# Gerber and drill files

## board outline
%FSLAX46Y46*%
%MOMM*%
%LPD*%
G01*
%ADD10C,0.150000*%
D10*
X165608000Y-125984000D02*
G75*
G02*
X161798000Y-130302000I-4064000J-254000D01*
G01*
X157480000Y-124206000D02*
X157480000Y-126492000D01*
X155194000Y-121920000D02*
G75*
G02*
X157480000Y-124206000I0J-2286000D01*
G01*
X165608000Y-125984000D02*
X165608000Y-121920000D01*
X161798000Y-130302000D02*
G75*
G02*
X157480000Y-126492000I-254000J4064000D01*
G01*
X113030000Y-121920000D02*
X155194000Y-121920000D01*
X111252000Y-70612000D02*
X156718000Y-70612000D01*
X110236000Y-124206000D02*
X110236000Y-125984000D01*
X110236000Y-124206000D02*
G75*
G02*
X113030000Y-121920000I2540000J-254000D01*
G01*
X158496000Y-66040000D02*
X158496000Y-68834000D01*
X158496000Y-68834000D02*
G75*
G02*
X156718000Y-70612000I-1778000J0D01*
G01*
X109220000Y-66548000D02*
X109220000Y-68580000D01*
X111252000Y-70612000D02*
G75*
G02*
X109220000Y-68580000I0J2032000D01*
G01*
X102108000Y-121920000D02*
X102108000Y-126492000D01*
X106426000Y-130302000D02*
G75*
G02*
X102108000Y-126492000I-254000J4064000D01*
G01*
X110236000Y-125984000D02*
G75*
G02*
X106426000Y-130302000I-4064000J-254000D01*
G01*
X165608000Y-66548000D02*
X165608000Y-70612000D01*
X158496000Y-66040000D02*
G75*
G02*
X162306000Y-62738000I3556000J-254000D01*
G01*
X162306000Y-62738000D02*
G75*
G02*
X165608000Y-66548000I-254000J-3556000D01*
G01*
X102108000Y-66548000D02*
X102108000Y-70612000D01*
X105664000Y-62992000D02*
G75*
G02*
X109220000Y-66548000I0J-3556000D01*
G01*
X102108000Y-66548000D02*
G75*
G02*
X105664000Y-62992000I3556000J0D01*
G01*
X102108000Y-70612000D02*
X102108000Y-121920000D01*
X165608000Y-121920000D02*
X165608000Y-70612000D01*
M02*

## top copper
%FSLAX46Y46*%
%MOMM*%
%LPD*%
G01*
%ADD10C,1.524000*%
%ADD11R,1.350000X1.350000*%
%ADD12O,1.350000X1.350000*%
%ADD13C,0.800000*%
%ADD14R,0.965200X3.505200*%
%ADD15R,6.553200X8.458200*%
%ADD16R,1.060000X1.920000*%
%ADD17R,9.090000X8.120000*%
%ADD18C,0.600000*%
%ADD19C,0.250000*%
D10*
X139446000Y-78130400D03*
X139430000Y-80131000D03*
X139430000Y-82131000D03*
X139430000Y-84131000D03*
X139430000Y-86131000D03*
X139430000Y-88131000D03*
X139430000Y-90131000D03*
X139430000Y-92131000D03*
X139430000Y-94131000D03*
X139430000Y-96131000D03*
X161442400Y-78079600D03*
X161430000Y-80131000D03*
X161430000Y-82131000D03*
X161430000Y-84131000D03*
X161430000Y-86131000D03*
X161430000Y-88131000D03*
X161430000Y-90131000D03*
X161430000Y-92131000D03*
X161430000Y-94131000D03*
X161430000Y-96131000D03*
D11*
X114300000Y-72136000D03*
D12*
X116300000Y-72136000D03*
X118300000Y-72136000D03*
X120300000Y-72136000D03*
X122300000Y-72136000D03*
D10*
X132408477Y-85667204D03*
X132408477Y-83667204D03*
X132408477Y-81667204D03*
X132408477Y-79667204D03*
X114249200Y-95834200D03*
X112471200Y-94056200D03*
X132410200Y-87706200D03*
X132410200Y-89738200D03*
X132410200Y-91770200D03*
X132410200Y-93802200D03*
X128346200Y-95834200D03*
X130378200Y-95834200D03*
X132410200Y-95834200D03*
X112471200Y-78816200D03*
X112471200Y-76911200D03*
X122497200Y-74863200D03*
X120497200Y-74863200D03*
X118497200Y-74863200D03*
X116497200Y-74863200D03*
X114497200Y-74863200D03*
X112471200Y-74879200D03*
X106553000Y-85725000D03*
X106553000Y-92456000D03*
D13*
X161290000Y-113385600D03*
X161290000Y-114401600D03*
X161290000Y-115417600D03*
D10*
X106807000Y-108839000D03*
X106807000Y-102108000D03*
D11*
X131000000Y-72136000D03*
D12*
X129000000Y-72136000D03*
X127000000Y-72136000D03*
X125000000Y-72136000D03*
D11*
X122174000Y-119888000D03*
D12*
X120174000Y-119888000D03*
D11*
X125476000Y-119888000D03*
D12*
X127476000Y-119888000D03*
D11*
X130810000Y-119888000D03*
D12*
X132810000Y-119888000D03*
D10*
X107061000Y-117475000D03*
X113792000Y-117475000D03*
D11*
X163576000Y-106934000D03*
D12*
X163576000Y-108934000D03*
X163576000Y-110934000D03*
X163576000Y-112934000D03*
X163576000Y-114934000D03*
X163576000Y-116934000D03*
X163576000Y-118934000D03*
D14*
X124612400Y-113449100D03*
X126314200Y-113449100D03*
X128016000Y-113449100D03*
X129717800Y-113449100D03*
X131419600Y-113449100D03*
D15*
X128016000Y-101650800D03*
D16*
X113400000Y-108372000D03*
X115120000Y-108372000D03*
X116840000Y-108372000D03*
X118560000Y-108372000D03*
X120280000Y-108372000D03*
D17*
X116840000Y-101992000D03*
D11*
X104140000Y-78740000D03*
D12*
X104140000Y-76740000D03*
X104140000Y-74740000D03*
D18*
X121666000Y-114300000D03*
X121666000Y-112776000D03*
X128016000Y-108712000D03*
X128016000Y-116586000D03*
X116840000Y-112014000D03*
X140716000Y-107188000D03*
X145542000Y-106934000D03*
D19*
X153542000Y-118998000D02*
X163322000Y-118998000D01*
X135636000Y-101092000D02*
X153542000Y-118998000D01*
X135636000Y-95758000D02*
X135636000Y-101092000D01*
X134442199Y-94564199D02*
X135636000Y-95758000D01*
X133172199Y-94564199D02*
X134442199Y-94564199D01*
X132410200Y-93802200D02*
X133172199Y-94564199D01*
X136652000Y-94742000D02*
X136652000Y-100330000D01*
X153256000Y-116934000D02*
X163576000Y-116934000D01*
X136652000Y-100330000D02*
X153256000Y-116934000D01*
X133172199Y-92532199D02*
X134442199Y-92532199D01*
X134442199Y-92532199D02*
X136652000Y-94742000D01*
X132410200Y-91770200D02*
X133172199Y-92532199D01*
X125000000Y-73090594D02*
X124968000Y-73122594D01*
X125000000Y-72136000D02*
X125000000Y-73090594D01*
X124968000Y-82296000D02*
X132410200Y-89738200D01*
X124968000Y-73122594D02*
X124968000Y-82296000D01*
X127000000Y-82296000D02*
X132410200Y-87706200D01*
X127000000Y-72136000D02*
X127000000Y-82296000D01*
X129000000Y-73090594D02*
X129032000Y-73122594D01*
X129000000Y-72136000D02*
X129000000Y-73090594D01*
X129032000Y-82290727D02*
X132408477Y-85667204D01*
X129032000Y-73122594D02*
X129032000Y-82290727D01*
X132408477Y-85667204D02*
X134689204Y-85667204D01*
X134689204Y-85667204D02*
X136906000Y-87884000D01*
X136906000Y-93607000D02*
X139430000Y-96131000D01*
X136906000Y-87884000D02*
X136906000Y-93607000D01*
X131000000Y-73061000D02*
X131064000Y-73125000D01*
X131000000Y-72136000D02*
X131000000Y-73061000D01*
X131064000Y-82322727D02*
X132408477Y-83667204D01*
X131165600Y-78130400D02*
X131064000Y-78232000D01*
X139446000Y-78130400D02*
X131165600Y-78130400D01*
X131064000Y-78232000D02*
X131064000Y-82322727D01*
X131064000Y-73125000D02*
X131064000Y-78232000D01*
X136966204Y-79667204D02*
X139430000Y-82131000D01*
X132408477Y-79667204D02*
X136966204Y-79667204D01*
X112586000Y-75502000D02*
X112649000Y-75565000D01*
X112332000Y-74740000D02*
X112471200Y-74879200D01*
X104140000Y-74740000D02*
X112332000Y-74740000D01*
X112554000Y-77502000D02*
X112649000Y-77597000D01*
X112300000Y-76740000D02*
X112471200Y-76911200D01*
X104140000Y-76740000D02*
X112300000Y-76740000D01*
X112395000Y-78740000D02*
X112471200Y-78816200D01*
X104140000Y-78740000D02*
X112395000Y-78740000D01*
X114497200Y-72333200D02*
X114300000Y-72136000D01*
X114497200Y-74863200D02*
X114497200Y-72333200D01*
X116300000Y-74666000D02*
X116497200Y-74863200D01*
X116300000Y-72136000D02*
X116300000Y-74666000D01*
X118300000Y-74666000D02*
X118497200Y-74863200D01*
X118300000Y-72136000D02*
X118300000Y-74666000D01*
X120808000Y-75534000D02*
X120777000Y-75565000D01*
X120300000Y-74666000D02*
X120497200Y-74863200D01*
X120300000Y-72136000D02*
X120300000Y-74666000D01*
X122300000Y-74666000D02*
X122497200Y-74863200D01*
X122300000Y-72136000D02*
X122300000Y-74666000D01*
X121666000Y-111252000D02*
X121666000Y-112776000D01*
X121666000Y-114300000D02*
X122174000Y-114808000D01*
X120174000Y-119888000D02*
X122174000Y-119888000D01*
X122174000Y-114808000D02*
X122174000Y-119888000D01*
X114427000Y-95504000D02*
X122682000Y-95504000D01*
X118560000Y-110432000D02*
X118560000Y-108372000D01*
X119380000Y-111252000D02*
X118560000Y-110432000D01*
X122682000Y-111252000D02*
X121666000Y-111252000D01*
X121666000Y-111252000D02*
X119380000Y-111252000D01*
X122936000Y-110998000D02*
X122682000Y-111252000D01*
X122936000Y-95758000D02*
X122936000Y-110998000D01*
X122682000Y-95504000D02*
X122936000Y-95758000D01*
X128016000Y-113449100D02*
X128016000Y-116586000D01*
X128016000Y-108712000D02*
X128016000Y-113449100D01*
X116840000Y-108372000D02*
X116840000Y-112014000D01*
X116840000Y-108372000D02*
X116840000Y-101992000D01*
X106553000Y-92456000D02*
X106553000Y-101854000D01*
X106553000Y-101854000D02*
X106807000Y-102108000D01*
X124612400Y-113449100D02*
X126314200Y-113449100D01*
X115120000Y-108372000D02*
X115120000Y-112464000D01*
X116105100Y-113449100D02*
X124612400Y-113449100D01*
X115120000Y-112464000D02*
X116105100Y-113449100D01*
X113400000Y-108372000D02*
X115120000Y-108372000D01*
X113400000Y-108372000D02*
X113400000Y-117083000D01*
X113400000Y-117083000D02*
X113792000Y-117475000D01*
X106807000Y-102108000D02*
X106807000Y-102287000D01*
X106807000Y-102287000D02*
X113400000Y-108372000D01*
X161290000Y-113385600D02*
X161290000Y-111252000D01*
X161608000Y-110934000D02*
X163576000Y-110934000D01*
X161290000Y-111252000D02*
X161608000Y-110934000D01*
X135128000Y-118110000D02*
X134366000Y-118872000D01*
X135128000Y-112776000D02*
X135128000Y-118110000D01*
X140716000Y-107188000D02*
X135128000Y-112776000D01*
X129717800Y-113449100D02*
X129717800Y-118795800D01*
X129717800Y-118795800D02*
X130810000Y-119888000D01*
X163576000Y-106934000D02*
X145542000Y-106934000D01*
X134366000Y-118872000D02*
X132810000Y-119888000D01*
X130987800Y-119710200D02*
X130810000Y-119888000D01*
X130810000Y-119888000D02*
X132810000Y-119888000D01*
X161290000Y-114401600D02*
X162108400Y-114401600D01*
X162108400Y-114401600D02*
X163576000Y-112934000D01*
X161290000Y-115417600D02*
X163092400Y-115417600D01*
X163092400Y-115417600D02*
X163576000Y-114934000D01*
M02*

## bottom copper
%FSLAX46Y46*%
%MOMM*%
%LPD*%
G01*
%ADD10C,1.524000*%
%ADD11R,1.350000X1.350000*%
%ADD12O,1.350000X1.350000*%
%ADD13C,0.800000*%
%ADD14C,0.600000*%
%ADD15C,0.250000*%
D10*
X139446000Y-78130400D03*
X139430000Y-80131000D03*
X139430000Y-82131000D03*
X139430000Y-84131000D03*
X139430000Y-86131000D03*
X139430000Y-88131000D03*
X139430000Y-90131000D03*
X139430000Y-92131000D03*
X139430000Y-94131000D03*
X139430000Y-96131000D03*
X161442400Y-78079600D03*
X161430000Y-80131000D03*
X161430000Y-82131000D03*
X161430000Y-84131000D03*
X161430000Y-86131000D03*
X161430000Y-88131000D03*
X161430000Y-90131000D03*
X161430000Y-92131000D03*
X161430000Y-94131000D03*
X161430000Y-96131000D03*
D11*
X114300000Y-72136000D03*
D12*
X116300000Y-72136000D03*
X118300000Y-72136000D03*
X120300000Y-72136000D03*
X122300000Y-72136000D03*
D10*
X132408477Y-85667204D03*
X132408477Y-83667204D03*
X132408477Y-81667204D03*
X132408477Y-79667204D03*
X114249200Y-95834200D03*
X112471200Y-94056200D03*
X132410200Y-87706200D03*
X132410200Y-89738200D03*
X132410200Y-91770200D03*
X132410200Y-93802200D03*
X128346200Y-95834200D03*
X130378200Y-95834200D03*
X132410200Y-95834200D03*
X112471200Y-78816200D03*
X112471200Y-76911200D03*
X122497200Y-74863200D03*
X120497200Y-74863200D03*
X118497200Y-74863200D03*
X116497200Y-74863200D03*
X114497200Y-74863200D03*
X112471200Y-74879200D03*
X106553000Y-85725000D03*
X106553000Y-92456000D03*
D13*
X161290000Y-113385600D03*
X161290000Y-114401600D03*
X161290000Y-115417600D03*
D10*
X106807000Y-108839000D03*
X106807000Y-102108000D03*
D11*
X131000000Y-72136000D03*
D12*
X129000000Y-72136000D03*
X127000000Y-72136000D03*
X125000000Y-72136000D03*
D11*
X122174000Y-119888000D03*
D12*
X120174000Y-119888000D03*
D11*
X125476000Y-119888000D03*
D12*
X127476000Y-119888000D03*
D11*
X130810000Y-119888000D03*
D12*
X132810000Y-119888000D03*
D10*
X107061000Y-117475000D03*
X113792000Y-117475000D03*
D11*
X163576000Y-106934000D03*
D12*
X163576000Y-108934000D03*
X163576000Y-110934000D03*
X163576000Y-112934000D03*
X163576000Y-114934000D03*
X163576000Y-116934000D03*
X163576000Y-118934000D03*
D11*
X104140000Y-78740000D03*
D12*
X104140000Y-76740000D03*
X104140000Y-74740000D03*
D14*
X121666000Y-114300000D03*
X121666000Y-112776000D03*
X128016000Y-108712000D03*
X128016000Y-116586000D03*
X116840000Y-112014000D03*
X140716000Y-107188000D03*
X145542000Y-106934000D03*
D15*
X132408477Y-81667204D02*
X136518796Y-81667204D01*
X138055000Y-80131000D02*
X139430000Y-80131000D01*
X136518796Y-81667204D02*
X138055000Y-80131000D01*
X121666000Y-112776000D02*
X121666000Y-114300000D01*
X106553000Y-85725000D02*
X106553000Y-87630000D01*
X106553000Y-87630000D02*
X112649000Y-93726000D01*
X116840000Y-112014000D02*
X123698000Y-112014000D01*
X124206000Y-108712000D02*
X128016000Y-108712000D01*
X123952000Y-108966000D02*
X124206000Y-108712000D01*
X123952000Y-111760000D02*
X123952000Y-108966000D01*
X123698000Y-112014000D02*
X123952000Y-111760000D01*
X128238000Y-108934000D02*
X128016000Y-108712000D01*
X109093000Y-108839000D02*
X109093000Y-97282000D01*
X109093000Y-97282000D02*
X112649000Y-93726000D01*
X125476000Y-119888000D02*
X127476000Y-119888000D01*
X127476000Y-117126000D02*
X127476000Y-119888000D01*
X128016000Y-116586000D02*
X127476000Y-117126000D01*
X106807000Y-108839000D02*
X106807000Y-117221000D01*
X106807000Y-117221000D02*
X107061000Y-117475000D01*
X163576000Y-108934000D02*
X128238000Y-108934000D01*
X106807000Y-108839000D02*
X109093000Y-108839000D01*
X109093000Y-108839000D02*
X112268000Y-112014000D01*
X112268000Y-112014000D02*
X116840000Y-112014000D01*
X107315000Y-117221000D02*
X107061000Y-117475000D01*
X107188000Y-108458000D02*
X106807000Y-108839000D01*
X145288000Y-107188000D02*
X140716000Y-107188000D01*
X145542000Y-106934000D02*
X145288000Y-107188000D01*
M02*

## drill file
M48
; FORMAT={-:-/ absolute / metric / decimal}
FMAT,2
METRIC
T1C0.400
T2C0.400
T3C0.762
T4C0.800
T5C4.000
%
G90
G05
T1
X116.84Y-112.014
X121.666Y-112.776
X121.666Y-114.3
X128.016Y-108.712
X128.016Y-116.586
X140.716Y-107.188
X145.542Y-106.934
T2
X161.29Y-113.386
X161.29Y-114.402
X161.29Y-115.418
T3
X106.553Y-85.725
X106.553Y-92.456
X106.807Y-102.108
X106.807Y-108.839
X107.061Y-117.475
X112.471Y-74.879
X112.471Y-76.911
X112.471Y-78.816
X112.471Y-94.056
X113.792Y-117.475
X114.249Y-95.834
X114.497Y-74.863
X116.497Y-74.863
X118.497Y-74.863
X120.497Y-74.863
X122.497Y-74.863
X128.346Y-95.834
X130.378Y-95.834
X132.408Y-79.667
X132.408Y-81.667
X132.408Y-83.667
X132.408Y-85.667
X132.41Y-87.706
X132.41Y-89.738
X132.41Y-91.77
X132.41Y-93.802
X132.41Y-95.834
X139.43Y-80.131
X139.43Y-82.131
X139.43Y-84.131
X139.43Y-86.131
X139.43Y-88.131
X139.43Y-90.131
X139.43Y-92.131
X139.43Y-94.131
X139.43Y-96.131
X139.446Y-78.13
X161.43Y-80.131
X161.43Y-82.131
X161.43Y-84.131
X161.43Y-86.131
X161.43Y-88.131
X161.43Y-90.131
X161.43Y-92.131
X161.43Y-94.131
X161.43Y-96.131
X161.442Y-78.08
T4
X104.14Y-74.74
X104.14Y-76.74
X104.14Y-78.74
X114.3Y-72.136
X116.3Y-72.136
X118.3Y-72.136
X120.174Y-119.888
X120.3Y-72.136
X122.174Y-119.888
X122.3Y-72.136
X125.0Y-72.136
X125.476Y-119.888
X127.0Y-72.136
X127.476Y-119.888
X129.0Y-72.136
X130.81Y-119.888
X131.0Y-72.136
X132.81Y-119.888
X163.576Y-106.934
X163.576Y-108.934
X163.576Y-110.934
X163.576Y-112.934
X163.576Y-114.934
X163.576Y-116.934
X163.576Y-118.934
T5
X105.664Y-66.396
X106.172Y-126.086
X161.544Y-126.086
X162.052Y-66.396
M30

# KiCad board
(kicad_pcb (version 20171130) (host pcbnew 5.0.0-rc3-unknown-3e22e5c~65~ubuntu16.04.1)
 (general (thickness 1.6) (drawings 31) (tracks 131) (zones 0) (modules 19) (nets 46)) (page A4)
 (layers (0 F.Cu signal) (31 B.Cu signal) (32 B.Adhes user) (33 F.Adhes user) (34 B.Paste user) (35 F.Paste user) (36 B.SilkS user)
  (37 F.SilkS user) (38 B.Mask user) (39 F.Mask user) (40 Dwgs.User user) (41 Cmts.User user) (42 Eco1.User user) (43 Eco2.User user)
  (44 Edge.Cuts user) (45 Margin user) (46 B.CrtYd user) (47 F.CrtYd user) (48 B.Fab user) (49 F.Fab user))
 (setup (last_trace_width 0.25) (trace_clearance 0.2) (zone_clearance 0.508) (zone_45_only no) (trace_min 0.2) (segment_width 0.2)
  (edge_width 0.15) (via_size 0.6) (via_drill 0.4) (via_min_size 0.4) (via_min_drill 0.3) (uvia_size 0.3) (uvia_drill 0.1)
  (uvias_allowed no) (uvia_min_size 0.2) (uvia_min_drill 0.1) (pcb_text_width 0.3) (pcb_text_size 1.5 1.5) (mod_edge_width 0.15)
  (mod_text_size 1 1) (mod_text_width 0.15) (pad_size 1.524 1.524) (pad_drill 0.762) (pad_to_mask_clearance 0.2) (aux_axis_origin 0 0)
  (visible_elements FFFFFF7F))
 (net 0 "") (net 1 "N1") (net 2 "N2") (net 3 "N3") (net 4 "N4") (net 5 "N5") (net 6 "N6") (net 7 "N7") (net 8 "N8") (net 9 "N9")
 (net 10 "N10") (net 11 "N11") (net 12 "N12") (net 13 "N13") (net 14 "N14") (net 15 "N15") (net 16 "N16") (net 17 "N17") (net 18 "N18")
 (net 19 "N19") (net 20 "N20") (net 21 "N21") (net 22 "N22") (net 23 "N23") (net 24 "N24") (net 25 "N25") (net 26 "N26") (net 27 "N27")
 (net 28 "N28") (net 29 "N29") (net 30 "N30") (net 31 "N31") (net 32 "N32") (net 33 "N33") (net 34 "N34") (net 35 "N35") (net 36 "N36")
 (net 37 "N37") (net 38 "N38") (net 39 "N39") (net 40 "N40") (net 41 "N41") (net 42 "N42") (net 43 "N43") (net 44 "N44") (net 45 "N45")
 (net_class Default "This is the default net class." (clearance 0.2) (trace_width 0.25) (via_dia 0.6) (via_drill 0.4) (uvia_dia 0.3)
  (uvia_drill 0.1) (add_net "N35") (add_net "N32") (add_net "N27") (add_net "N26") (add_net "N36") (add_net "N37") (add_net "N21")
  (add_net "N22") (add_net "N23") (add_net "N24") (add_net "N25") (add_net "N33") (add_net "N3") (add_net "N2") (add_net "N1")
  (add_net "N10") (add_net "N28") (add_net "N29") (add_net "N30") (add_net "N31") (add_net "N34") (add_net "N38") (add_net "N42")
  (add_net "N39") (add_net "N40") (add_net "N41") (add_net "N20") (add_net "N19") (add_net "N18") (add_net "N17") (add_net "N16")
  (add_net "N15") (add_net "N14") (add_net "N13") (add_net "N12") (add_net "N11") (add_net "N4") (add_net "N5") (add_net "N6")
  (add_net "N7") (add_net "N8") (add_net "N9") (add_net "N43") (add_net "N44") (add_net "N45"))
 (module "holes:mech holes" (layer F.Cu) (at 162.052 129.286)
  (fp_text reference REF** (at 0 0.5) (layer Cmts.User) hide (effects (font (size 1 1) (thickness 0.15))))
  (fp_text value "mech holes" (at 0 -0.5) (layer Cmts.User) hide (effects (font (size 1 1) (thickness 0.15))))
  (pad "" np_thru_hole circle (at -0.508 -3.2004) (size 4 4) (drill 4) (layers *.Cu *.Mask)))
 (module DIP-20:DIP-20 (layer F.Cu) (at 138.176 104.14)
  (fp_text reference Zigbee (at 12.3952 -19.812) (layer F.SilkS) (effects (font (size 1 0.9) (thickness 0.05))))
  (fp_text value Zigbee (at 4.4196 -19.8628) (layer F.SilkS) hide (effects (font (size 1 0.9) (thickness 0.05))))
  (pad 1 thru_hole circle (at 1.27 -26.0096) (size 1.524 1.524) (drill 0.762) (layers *.Cu *.Mask F.SilkS) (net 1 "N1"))
  (pad 2 thru_hole circle (at 1.254 -24.009) (size 1.524 1.524) (drill 0.762) (layers *.Cu *.Mask F.SilkS) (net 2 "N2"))
  (pad 3 thru_hole circle (at 1.254 -22.009) (size 1.524 1.524) (drill 0.762) (layers *.Cu *.Mask F.SilkS) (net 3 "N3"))
  (pad 4 thru_hole circle (at 1.254 -20.009) (size 1.524 1.524) (drill 0.762) (layers *.Cu *.Mask F.SilkS) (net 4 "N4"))
  (pad 5 thru_hole circle (at 1.254 -18.009) (size 1.524 1.524) (drill 0.762) (layers *.Cu *.Mask F.SilkS) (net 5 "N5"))
  (pad 6 thru_hole circle (at 1.254 -16.009) (size 1.524 1.524) (drill 0.762) (layers *.Cu *.Mask F.SilkS) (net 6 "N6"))
  (pad 7 thru_hole circle (at 1.254 -14.009) (size 1.524 1.524) (drill 0.762) (layers *.Cu *.Mask F.SilkS) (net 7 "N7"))
  (pad 8 thru_hole circle (at 1.254 -12.009) (size 1.524 1.524) (drill 0.762) (layers *.Cu *.Mask F.SilkS) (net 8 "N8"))
  (pad 9 thru_hole circle (at 1.254 -10.009) (size 1.524 1.524) (drill 0.762) (layers *.Cu *.Mask F.SilkS) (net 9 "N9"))
  (pad 10 thru_hole circle (at 1.254 -8.009) (size 1.524 1.524) (drill 0.762) (layers *.Cu *.Mask F.SilkS) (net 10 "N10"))
  (pad 20 thru_hole circle (at 23.2664 -26.0604) (size 1.524 1.524) (drill 0.762) (layers *.Cu *.Mask F.SilkS) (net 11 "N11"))
  (pad 19 thru_hole circle (at 23.254 -24.009) (size 1.524 1.524) (drill 0.762) (layers *.Cu *.Mask F.SilkS) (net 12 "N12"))
  (pad 18 thru_hole circle (at 23.254 -22.009) (size 1.524 1.524) (drill 0.762) (layers *.Cu *.Mask F.SilkS) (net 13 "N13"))
  (pad 17 thru_hole circle (at 23.254 -20.009) (size 1.524 1.524) (drill 0.762) (layers *.Cu *.Mask F.SilkS) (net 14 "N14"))
  (pad 16 thru_hole circle (at 23.254 -18.009) (size 1.524 1.524) (drill 0.762) (layers *.Cu *.Mask F.SilkS) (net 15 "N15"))
  (pad 15 thru_hole circle (at 23.254 -16.009) (size 1.524 1.524) (drill 0.762) (layers *.Cu *.Mask F.SilkS) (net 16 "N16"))
  (pad 14 thru_hole circle (at 23.254 -14.009) (size 1.524 1.524) (drill 0.762) (layers *.Cu *.Mask F.SilkS) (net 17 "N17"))
  (pad 13 thru_hole circle (at 23.254 -12.009) (size 1.524 1.524) (drill 0.762) (layers *.Cu *.Mask F.SilkS) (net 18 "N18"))
  (pad 12 thru_hole circle (at 23.254 -10.009) (size 1.524 1.524) (drill 0.762) (layers *.Cu *.Mask F.SilkS) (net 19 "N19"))
  (pad 11 thru_hole circle (at 23.254 -8.009) (size 1.524 1.524) (drill 0.762) (layers *.Cu *.Mask F.SilkS) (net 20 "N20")))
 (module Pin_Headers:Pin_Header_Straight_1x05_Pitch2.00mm (layer F.Cu) (at 114.3 72.136 90)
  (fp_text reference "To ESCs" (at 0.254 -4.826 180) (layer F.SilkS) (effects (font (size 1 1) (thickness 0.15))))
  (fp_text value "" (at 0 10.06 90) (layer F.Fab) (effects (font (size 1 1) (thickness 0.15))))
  (pad 1 thru_hole rect (at 0 0 90) (size 1.35 1.35) (drill 0.8) (layers *.Cu *.Mask) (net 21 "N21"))
  (pad 2 thru_hole oval (at 0 2 90) (size 1.35 1.35) (drill 0.8) (layers *.Cu *.Mask) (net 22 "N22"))
  (pad 3 thru_hole oval (at 0 4 90) (size 1.35 1.35) (drill 0.8) (layers *.Cu *.Mask) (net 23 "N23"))
  (pad 4 thru_hole oval (at 0 6 90) (size 1.35 1.35) (drill 0.8) (layers *.Cu *.Mask) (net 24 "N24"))
  (pad 5 thru_hole oval (at 0 8 90) (size 1.35 1.35) (drill 0.8) (layers *.Cu *.Mask) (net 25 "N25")))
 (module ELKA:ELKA (layer F.Cu) (at 121.666 85.852)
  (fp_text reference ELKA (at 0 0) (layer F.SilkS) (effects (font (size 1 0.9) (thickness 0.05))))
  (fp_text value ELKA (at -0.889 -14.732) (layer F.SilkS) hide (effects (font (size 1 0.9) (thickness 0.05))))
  (pad D thru_hole circle (at 10.742477 -0.184796) (size 1.524 1.524) (drill 0.762) (layers *.Cu *.Mask B.SilkS) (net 10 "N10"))
  (pad C thru_hole circle (at 10.742477 -2.184796) (size 1.524 1.524) (drill 0.762) (layers *.Cu *.Mask B.SilkS) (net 1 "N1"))
  (pad B thru_hole circle (at 10.742477 -4.184796) (size 1.524 1.524) (drill 0.762) (layers *.Cu *.Mask B.SilkS) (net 2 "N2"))
  (pad A thru_hole circle (at 10.742477 -6.184796) (size 1.524 1.524) (drill 0.762) (layers *.Cu *.Mask B.SilkS) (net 3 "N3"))
  (pad 12 thru_hole circle (at -7.4168 9.9822) (size 1.524 1.524) (drill 0.762) (layers *.Cu *.Mask B.SilkS) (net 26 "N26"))
  (pad 11 thru_hole circle (at -9.1948 8.2042 270) (size 1.524 1.524) (drill 0.762) (layers *.Cu *.Mask B.SilkS) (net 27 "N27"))
  (pad E thru_hole circle (at 10.7442 1.8542 270) (size 1.524 1.524) (drill 0.762) (layers *.Cu *.Mask B.SilkS) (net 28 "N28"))
  (pad F thru_hole circle (at 10.7442 3.8862 270) (size 1.524 1.524) (drill 0.762) (layers *.Cu *.Mask B.SilkS) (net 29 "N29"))
  (pad G thru_hole circle (at 10.7442 5.9182 270) (size 1.524 1.524) (drill 0.762) (layers *.Cu *.Mask B.SilkS) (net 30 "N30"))
  (pad H thru_hole circle (at 10.7442 7.9502 270) (size 1.524 1.524) (drill 0.762) (layers *.Cu *.Mask B.SilkS) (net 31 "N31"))
  (pad 10 thru_hole circle (at 6.6802 9.9822 270) (size 1.524 1.524) (drill 0.762) (layers *.Cu *.Mask B.SilkS) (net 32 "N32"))
  (pad 9 thru_hole circle (at 8.7122 9.9822 270) (size 1.524 1.524) (drill 0.762) (layers *.Cu *.Mask B.SilkS) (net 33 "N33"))
  (pad I thru_hole circle (at 10.7442 9.9822 270) (size 1.524 1.524) (drill 0.762) (layers *.Cu *.Mask B.SilkS) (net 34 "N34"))
  (pad 1 thru_hole circle (at -9.1948 -7.0358 270) (size 1.524 1.524) (drill 0.762) (layers *.Cu *.Mask B.SilkS) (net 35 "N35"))
  (pad 2 thru_hole circle (at -9.1948 -8.9408 270) (size 1.524 1.524) (drill 0.762) (layers *.Cu *.Mask B.SilkS) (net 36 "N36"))
  (pad 8 thru_hole circle (at 0.8312 -10.9888 270) (size 1.524 1.524) (drill 0.762) (layers *.Cu *.Mask B.SilkS) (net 25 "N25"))
  (pad 7 thru_hole circle (at -1.1688 -10.9888 270) (size 1.524 1.524) (drill 0.762) (layers *.Cu *.Mask B.SilkS) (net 24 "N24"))
  (pad 6 thru_hole circle (at -3.1688 -10.9888 270) (size 1.524 1.524) (drill 0.762) (layers *.Cu *.Mask B.SilkS) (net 23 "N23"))
  (pad 5 thru_hole circle (at -5.1688 -10.9888 270) (size 1.524 1.524) (drill 0.762) (layers *.Cu *.Mask B.SilkS) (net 22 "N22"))
  (pad 4 thru_hole circle (at -7.1688 -10.9888 270) (size 1.524 1.524) (drill 0.762) (layers *.Cu *.Mask B.SilkS) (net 21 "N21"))
  (pad 3 thru_hole circle (at -9.1948 -10.9728 270) (size 1.524 1.524) (drill 0.762) (layers *.Cu *.Mask B.SilkS) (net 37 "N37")))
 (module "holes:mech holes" (layer F.Cu) (at 106.172 69.596)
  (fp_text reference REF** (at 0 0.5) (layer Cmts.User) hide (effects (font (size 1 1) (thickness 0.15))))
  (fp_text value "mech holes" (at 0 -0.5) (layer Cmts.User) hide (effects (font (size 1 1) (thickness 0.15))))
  (pad "" np_thru_hole circle (at -0.508 -3.2004) (size 4 4) (drill 4) (layers *.Cu *.Mask)))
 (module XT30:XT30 (layer F.Cu) (at 112.522 87.122 270)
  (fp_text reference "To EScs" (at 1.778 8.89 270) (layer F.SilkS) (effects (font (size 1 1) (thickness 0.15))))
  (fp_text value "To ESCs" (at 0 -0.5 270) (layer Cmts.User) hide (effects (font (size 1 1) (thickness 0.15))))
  (pad 1 thru_hole circle (at -1.397 5.969 270) (size 1.524 1.524) (drill 0.762) (layers *.Cu *.Mask) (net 27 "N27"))
  (pad 2 thru_hole circle (at 5.334 5.969 270) (size 1.524 1.524) (drill 0.762) (layers *.Cu *.Mask) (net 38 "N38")))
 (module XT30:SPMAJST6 (layer F.Cu) (at 164.084 115.316 270)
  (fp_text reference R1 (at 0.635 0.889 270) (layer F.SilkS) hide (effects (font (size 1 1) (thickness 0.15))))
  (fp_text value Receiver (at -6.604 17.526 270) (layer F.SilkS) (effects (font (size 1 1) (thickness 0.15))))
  (pad 1 thru_hole circle (at -1.9304 2.794 270) (size 0.8 0.8) (drill 0.4) (layers *.Cu *.Mask) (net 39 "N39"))
  (pad 2 thru_hole circle (at -0.9144 2.794 270) (size 0.8 0.8) (drill 0.4) (layers *.Cu *.Mask) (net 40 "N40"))
  (pad 3 thru_hole circle (at 0.1016 2.794 270) (size 0.8 0.8) (drill 0.4) (layers *.Cu *.Mask) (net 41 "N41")))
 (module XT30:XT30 (layer F.Cu) (at 100.838 107.442 90)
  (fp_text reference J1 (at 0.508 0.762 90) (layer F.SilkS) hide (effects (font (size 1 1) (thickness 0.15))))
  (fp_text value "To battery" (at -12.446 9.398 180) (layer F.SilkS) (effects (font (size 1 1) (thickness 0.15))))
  (pad 1 thru_hole circle (at -1.397 5.969 90) (size 1.524 1.524) (drill 0.762) (layers *.Cu *.Mask) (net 27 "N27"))
  (pad 2 thru_hole circle (at 5.334 5.969 90) (size 1.524 1.524) (drill 0.762) (layers *.Cu *.Mask) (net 38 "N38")))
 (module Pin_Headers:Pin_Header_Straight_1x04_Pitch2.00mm (layer F.Cu) (at 131 72.136 270)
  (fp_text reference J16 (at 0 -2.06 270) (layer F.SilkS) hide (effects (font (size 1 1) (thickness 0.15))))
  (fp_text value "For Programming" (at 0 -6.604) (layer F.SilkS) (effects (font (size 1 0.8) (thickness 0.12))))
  (pad 1 thru_hole rect (at 0 0 270) (size 1.35 1.35) (drill 0.8) (layers *.Cu *.Mask) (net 1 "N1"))
  (pad 2 thru_hole oval (at 0 2 270) (size 1.35 1.35) (drill 0.8) (layers *.Cu *.Mask) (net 10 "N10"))
  (pad 3 thru_hole oval (at 0 4 270) (size 1.35 1.35) (drill 0.8) (layers *.Cu *.Mask) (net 28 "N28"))
  (pad 4 thru_hole oval (at 0 6 270) (size 1.35 1.35) (drill 0.8) (layers *.Cu *.Mask) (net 29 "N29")))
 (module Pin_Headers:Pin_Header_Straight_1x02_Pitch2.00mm (layer F.Cu) (at 122.174 119.888 270)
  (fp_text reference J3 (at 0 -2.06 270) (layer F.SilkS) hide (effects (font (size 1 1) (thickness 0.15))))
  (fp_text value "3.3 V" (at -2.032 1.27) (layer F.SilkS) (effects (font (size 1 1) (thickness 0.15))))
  (pad 1 thru_hole rect (at 0 0 270) (size 1.35 1.35) (drill 0.8) (layers *.Cu *.Mask) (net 26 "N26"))
  (pad 2 thru_hole oval (at 0 2 270) (size 1.35 1.35) (drill 0.8) (layers *.Cu *.Mask) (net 26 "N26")))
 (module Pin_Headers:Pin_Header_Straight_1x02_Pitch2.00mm (layer F.Cu) (at 125.476 119.888 90)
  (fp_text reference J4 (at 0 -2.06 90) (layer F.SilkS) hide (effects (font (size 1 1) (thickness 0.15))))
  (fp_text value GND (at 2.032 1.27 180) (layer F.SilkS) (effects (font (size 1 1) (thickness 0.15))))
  (pad 1 thru_hole rect (at 0 0 90) (size 1.35 1.35) (drill 0.8) (layers *.Cu *.Mask) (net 27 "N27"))
  (pad 2 thru_hole oval (at 0 2 90) (size 1.35 1.35) (drill 0.8) (layers *.Cu *.Mask) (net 27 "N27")))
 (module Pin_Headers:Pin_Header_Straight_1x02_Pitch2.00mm (layer F.Cu) (at 130.81 119.888 90)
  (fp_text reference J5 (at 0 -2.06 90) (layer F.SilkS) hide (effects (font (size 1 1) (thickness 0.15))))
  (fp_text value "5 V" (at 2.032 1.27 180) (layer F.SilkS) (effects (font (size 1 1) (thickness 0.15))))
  (pad 1 thru_hole rect (at 0 0 90) (size 1.35 1.35) (drill 0.8) (layers *.Cu *.Mask) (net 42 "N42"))
  (pad 2 thru_hole oval (at 0 2 90) (size 1.35 1.35) (drill 0.8) (layers *.Cu *.Mask) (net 42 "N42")))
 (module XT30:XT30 (layer F.Cu) (at 108.458 111.506)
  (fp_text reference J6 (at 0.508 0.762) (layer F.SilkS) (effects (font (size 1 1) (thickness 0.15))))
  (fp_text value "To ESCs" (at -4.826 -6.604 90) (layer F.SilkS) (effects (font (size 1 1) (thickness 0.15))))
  (pad 1 thru_hole circle (at -1.397 5.969) (size 1.524 1.524) (drill 0.762) (layers *.Cu *.Mask) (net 27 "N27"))
  (pad 2 thru_hole circle (at 5.334 5.969) (size 1.524 1.524) (drill 0.762) (layers *.Cu *.Mask) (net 38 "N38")))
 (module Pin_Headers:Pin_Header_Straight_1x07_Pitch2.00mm (layer F.Cu) (at 163.576 106.934)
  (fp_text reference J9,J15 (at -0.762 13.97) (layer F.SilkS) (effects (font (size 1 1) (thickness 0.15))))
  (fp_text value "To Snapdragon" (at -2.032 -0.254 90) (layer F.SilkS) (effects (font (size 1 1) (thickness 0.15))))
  (pad 1 thru_hole rect (at 0 0) (size 1.35 1.35) (drill 0.8) (layers *.Cu *.Mask) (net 42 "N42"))
  (pad 2 thru_hole oval (at 0 2) (size 1.35 1.35) (drill 0.8) (layers *.Cu *.Mask) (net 27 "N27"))
  (pad 3 thru_hole oval (at 0 4) (size 1.35 1.35) (drill 0.8) (layers *.Cu *.Mask) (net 39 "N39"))
  (pad 4 thru_hole oval (at 0 6) (size 1.35 1.35) (drill 0.8) (layers *.Cu *.Mask) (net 40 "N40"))
  (pad 5 thru_hole oval (at 0 8) (size 1.35 1.35) (drill 0.8) (layers *.Cu *.Mask) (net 41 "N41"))
  (pad 6 thru_hole oval (at 0 10) (size 1.35 1.35) (drill 0.8) (layers *.Cu *.Mask) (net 30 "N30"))
  (pad 7 thru_hole oval (at 0 12) (size 1.35 1.35) (drill 0.8) (layers *.Cu *.Mask) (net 31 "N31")))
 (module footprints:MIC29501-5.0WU (layer F.Cu) (at 128.016 104.394)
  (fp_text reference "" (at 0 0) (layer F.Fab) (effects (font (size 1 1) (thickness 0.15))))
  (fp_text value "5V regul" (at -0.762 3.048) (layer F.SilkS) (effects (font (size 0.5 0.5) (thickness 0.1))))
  (pad 1 smd rect (at -3.4036 9.0551) (size 0.9652 3.5052) (layers F.Cu F.Paste F.Mask) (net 38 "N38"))
  (pad 2 smd rect (at -1.7018 9.0551) (size 0.9652 3.5052) (layers F.Cu F.Paste F.Mask) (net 38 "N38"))
  (pad 3 smd rect (at 0 9.0551) (size 0.9652 3.5052) (layers F.Cu F.Paste F.Mask) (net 27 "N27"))
  (pad 4 smd rect (at 1.7018 9.0551) (size 0.9652 3.5052) (layers F.Cu F.Paste F.Mask) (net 42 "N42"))
  (pad 5 smd rect (at 3.4036 9.0551) (size 0.9652 3.5052) (layers F.Cu F.Paste F.Mask) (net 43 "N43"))
  (pad 6 smd rect (at 0 -2.7432) (size 6.5532 8.4582) (layers F.Cu F.Paste F.Mask) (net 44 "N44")))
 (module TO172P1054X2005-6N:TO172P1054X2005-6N (layer F.Cu) (at 116.84 103.632)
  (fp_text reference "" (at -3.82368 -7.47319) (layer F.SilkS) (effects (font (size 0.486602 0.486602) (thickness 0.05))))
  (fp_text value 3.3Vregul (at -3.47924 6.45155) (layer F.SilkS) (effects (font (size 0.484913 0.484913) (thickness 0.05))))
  (pad 1 smd rect (at -3.44 4.74 90) (size 1.92 1.06) (layers F.Cu F.Paste F.Mask) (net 38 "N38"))
  (pad 2 smd rect (at -1.72 4.74 90) (size 1.92 1.06) (layers F.Cu F.Paste F.Mask) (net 38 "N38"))
  (pad 3 smd rect (at 0 4.74 90) (size 1.92 1.06) (layers F.Cu F.Paste F.Mask) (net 27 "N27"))
  (pad 4 smd rect (at 1.72 4.74 90) (size 1.92 1.06) (layers F.Cu F.Paste F.Mask) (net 26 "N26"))
  (pad 5 smd rect (at 3.44 4.74 90) (size 1.92 1.06) (layers F.Cu F.Paste F.Mask) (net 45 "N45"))
  (pad 6 smd rect (at 0 -1.64 90) (size 8.12 9.09) (layers F.Cu F.Paste F.Mask) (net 27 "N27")))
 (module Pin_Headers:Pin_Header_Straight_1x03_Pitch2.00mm (layer F.Cu) (at 104.14 78.74 180)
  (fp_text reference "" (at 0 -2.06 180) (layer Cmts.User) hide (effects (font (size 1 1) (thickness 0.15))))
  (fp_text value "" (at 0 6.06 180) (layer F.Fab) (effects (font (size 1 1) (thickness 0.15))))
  (pad 1 thru_hole rect (at 0 0 180) (size 1.35 1.35) (drill 0.8) (layers *.Cu *.Mask) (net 35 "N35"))
  (pad 2 thru_hole oval (at 0 2 180) (size 1.35 1.35) (drill 0.8) (layers *.Cu *.Mask) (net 36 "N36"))
  (pad 3 thru_hole oval (at 0 4 180) (size 1.35 1.35) (drill 0.8) (layers *.Cu *.Mask) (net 37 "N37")))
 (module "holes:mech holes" (layer F.Cu) (at 162.56 69.596)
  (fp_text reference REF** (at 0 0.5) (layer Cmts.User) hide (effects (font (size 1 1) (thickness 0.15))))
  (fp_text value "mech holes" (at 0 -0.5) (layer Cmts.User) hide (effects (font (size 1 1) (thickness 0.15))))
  (pad "" np_thru_hole circle (at -0.508 -3.2004) (size 4 4) (drill 4) (layers *.Cu *.Mask)))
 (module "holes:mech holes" (layer F.Cu) (at 106.68 129.286)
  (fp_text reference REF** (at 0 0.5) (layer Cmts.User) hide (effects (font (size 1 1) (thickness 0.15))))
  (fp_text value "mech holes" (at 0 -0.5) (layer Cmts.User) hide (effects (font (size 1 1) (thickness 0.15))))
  (pad "" np_thru_hole circle (at -0.508 -3.2004) (size 4 4) (drill 4) (layers *.Cu *.Mask)))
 (gr_arc (start 161.544 126.238) (end 165.608 125.984) (angle 90) (layer Edge.Cuts) (width 0.15))
 (gr_line (start 157.48 124.206) (end 157.48 126.492) (angle 90) (layer Edge.Cuts) (width 0.15))
 (gr_arc (start 155.194 124.206) (end 155.194 121.92) (angle 90) (layer Edge.Cuts) (width 0.15))
 (gr_line (start 165.608 125.984) (end 165.608 121.92) (angle 90) (layer Edge.Cuts) (width 0.15))
 (gr_arc (start 161.544 126.238) (end 161.798 130.302) (angle 90) (layer Edge.Cuts) (width 0.15))
 (gr_line (start 113.03 121.92) (end 155.194 121.92) (angle 90) (layer Edge.Cuts) (width 0.15))
 (gr_line (start 111.252 70.612) (end 156.718 70.612) (angle 90) (layer Edge.Cuts) (width 0.15))
 (gr_line (start 110.236 124.206) (end 110.236 125.984) (angle 90) (layer Edge.Cuts) (width 0.15))
 (gr_arc (start 112.776 124.46) (end 110.236 124.206) (angle 90) (layer Edge.Cuts) (width 0.15))
 (gr_line (start 158.496 66.04) (end 158.496 68.834) (angle 90) (layer Edge.Cuts) (width 0.15))
 (gr_arc (start 156.718 68.834) (end 158.496 68.834) (angle 90) (layer Edge.Cuts) (width 0.15))
 (gr_line (start 109.22 66.548) (end 109.22 68.58) (angle 90) (layer Edge.Cuts) (width 0.15))
 (gr_arc (start 111.252 68.58) (end 111.252 70.612) (angle 90) (layer Edge.Cuts) (width 0.15))
 (gr_line (start 102.108 121.92) (end 102.108 126.492) (angle 90) (layer Edge.Cuts) (width 0.15))
 (gr_arc (start 106.172 126.238) (end 106.426 130.302) (angle 90) (layer Edge.Cuts) (width 0.15))
 (gr_arc (start 106.172 126.238) (end 110.236 125.984) (angle 90) (layer Edge.Cuts) (width 0.15))
 (gr_line (start 165.608 66.548) (end 165.608 70.612) (angle 90) (layer Edge.Cuts) (width 0.15))
 (gr_arc (start 162.052 66.294) (end 158.496 66.04) (angle 90) (layer Edge.Cuts) (width 0.15))
 (gr_arc (start 162.052 66.294) (end 162.306 62.738) (angle 90) (layer Edge.Cuts) (width 0.15))
 (gr_line (start 102.108 66.548) (end 102.108 70.612) (angle 90) (layer Edge.Cuts) (width 0.15))
 (gr_arc (start 105.664 66.548) (end 105.664 62.992) (angle 90) (layer Edge.Cuts) (width 0.15))
 (gr_arc (start 105.664 66.548) (end 102.108 66.548) (angle 90) (layer Edge.Cuts) (width 0.15))
 (gr_line (start 102.108 70.612) (end 102.108 121.92) (angle 90) (layer Edge.Cuts) (width 0.15))
 (gr_line (start 165.608 121.92) (end 165.608 70.612) (angle 90) (layer Edge.Cuts) (width 0.15))
 (segment (start 153.542 118.998) (end 163.322 118.998) (width 0.25) (layer F.Cu) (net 31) (status 20))
 (segment (start 135.636 101.092) (end 153.542 118.998) (width 0.25) (layer F.Cu) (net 31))
 (segment (start 135.636 95.758) (end 135.636 101.092) (width 0.25) (layer F.Cu) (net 31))
 (segment (start 134.442199 94.564199) (end 135.636 95.758) (width 0.25) (layer F.Cu) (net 31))
 (segment (start 133.172199 94.564199) (end 134.442199 94.564199) (width 0.25) (layer F.Cu) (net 31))
 (segment (start 132.4102 93.8022) (end 133.172199 94.564199) (width 0.25) (layer F.Cu) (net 31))
 (segment (start 136.652 94.742) (end 136.652 100.33) (width 0.25) (layer F.Cu) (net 30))
 (segment (start 153.256 116.934) (end 163.576 116.934) (width 0.25) (layer F.Cu) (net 30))
 (segment (start 136.652 100.33) (end 153.256 116.934) (width 0.25) (layer F.Cu) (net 30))
 (segment (start 133.172199 92.532199) (end 134.442199 92.532199) (width 0.25) (layer F.Cu) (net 30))
 (segment (start 134.442199 92.532199) (end 136.652 94.742) (width 0.25) (layer F.Cu) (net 30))
 (segment (start 132.4102 91.7702) (end 133.172199 92.532199) (width 0.25) (layer F.Cu) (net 30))
 (segment (start 125 73.090594) (end 124.968 73.122594) (width 0.25) (layer F.Cu) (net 29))
 (segment (start 125 72.136) (end 125 73.090594) (width 0.25) (layer F.Cu) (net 29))
 (segment (start 124.968 82.296) (end 132.4102 89.7382) (width 0.25) (layer F.Cu) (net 29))
 (segment (start 124.968 73.122594) (end 124.968 82.296) (width 0.25) (layer F.Cu) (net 29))
 (segment (start 127 82.296) (end 132.4102 87.7062) (width 0.25) (layer F.Cu) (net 28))
 (segment (start 127 72.136) (end 127 82.296) (width 0.25) (layer F.Cu) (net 28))
 (segment (start 129 73.090594) (end 129.032 73.122594) (width 0.25) (layer F.Cu) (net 10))
 (segment (start 129 72.136) (end 129 73.090594) (width 0.25) (layer F.Cu) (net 10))
 (segment (start 129.032 82.290727) (end 132.408477 85.667204) (width 0.25) (layer F.Cu) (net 10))
 (segment (start 129.032 73.122594) (end 129.032 82.290727) (width 0.25) (layer F.Cu) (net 10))
 (segment (start 132.408477 85.667204) (end 134.689204 85.667204) (width 0.25) (layer F.Cu) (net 10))
 (segment (start 134.689204 85.667204) (end 136.906 87.884) (width 0.25) (layer F.Cu) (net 10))
 (segment (start 136.906 93.607) (end 139.43 96.131) (width 0.25) (layer F.Cu) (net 10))
 (segment (start 136.906 87.884) (end 136.906 93.607) (width 0.25) (layer F.Cu) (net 10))
 (segment (start 131 73.061) (end 131.064 73.125) (width 0.25) (layer F.Cu) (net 1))
 (segment (start 131 72.136) (end 131 73.061) (width 0.25) (layer F.Cu) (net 1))
 (segment (start 131.064 82.322727) (end 132.408477 83.667204) (width 0.25) (layer F.Cu) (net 1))
 (segment (start 131.1656 78.1304) (end 131.064 78.232) (width 0.25) (layer F.Cu) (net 1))
 (segment (start 139.446 78.1304) (end 131.1656 78.1304) (width 0.25) (layer F.Cu) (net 1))
 (segment (start 131.064 78.232) (end 131.064 82.322727) (width 0.25) (layer F.Cu) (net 1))
 (segment (start 131.064 73.125) (end 131.064 78.232) (width 0.25) (layer F.Cu) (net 1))
 (segment (start 132.408477 81.667204) (end 136.518796 81.667204) (width 0.25) (layer B.Cu) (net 2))
 (segment (start 138.055 80.131) (end 139.43 80.131) (width 0.25) (layer B.Cu) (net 2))
 (segment (start 136.518796 81.667204) (end 138.055 80.131) (width 0.25) (layer B.Cu) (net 2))
 (segment (start 136.966204 79.667204) (end 139.43 82.131) (width 0.25) (layer F.Cu) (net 3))
 (segment (start 132.408477 79.667204) (end 136.966204 79.667204) (width 0.25) (layer F.Cu) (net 3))
 (segment (start 112.586 75.502) (end 112.649 75.565) (width 0.25) (layer F.Cu) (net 37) (status 30))
 (segment (start 112.332 74.74) (end 112.4712 74.8792) (width 0.25) (layer F.Cu) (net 37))
 (segment (start 104.14 74.74) (end 112.332 74.74) (width 0.25) (layer F.Cu) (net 37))
 (segment (start 112.554 77.502) (end 112.649 77.597) (width 0.25) (layer F.Cu) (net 36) (status 30))
 (segment (start 112.3 76.74) (end 112.4712 76.9112) (width 0.25) (layer F.Cu) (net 36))
 (segment (start 104.14 76.74) (end 112.3 76.74) (width 0.25) (layer F.Cu) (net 36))
 (segment (start 112.395 78.74) (end 112.4712 78.8162) (width 0.25) (layer F.Cu) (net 35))
 (segment (start 104.14 78.74) (end 112.395 78.74) (width 0.25) (layer F.Cu) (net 35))
 (segment (start 114.4972 72.3332) (end 114.3 72.136) (width 0.25) (layer F.Cu) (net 21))
 (segment (start 114.4972 74.8632) (end 114.4972 72.3332) (width 0.25) (layer F.Cu) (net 21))
 (segment (start 116.3 74.666) (end 116.4972 74.8632) (width 0.25) (layer F.Cu) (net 22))
 (segment (start 116.3 72.136) (end 116.3 74.666) (width 0.25) (layer F.Cu) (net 22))
 (segment (start 118.3 74.666) (end 118.4972 74.8632) (width 0.25) (layer F.Cu) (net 23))
 (segment (start 118.3 72.136) (end 118.3 74.666) (width 0.25) (layer F.Cu) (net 23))
 (segment (start 120.808 75.534) (end 120.777 75.565) (width 0.25) (layer F.Cu) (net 24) (status 30))
 (segment (start 120.3 74.666) (end 120.4972 74.8632) (width 0.25) (layer F.Cu) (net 24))
 (segment (start 120.3 72.136) (end 120.3 74.666) (width 0.25) (layer F.Cu) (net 24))
 (segment (start 122.3 74.666) (end 122.4972 74.8632) (width 0.25) (layer F.Cu) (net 25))
 (segment (start 122.3 72.136) (end 122.3 74.666) (width 0.25) (layer F.Cu) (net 25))
 (segment (start 121.666 111.252) (end 121.666 112.776) (width 0.25) (layer F.Cu) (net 26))
 (segment (start 121.666 114.3) (end 122.174 114.808) (width 0.25) (layer F.Cu) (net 26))
 (via (at 121.666 114.3) (size 0.6) (drill 0.4) (layers F.Cu B.Cu) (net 26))
 (segment (start 121.666 112.776) (end 121.666 114.3) (width 0.25) (layer B.Cu) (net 26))
 (via (at 121.666 112.776) (size 0.6) (drill 0.4) (layers F.Cu B.Cu) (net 26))
 (segment (start 120.174 119.888) (end 122.174 119.888) (width 0.25) (layer F.Cu) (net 26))
 (segment (start 122.174 114.808) (end 122.174 119.888) (width 0.25) (layer F.Cu) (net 26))
 (segment (start 114.427 95.504) (end 122.682 95.504) (width 0.25) (layer F.Cu) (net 26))
 (segment (start 118.56 110.432) (end 118.56 108.372) (width 0.25) (layer F.Cu) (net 26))
 (segment (start 119.38 111.252) (end 118.56 110.432) (width 0.25) (layer F.Cu) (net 26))
 (segment (start 122.682 111.252) (end 121.666 111.252) (width 0.25) (layer F.Cu) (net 26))
 (segment (start 121.666 111.252) (end 119.38 111.252) (width 0.25) (layer F.Cu) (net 26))
 (segment (start 122.936 110.998) (end 122.682 111.252) (width 0.25) (layer F.Cu) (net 26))
 (segment (start 122.936 95.758) (end 122.936 110.998) (width 0.25) (layer F.Cu) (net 26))
 (segment (start 122.682 95.504) (end 122.936 95.758) (width 0.25) (layer F.Cu) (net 26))
 (segment (start 106.553 85.725) (end 106.553 87.63) (width 0.25) (layer B.Cu) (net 27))
 (segment (start 106.553 87.63) (end 112.649 93.726) (width 0.25) (layer B.Cu) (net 27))
 (segment (start 116.84 112.014) (end 123.698 112.014) (width 0.25) (layer B.Cu) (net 27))
 (segment (start 124.206 108.712) (end 128.016 108.712) (width 0.25) (layer B.Cu) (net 27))
 (segment (start 123.952 108.966) (end 124.206 108.712) (width 0.25) (layer B.Cu) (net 27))
 (segment (start 123.952 111.76) (end 123.952 108.966) (width 0.25) (layer B.Cu) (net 27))
 (segment (start 123.698 112.014) (end 123.952 111.76) (width 0.25) (layer B.Cu) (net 27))
 (segment (start 128.238 108.934) (end 128.016 108.712) (width 0.25) (layer B.Cu) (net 27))
 (via (at 128.016 108.712) (size 0.6) (drill 0.4) (layers F.Cu B.Cu) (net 27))
 (segment (start 109.093 108.839) (end 109.093 97.282) (width 0.25) (layer B.Cu) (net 27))
 (segment (start 109.093 97.282) (end 112.649 93.726) (width 0.25) (layer B.Cu) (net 27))
 (segment (start 125.476 119.888) (end 127.476 119.888) (width 0.25) (layer B.Cu) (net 27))
 (segment (start 128.016 113.4491) (end 128.016 116.586) (width 0.25) (layer F.Cu) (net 27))
 (segment (start 127.476 117.126) (end 127.476 119.888) (width 0.25) (layer B.Cu) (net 27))
 (segment (start 128.016 116.586) (end 127.476 117.126) (width 0.25) (layer B.Cu) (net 27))
 (via (at 128.016 116.586) (size 0.6) (drill 0.4) (layers F.Cu B.Cu) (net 27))
 (segment (start 106.807 108.839) (end 106.807 117.221) (width 0.25) (layer B.Cu) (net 27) (status 10))
 (segment (start 106.807 117.221) (end 107.061 117.475) (width 0.25) (layer B.Cu) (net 27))
 (segment (start 163.576 108.934) (end 128.238 108.934) (width 0.25) (layer B.Cu) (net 27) (status 10))
 (segment (start 128.016 108.712) (end 128.016 113.4491) (width 0.25) (layer F.Cu) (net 27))
 (segment (start 116.84 108.372) (end 116.84 112.014) (width 0.25) (layer F.Cu) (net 27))
 (via (at 116.84 112.014) (size 0.6) (drill 0.4) (layers F.Cu B.Cu) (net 27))
 (segment (start 106.807 108.839) (end 109.093 108.839) (width 0.25) (layer B.Cu) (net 27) (status 10))
 (segment (start 109.093 108.839) (end 112.268 112.014) (width 0.25) (layer B.Cu) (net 27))
 (segment (start 112.268 112.014) (end 116.84 112.014) (width 0.25) (layer B.Cu) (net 27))
 (segment (start 107.315 117.221) (end 107.061 117.475) (width 0.25) (layer B.Cu) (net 27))
 (segment (start 107.188 108.458) (end 106.807 108.839) (width 0.25) (layer B.Cu) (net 27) (status 30))
 (segment (start 116.84 108.372) (end 116.84 101.992) (width 0.25) (layer F.Cu) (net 27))
 (segment (start 106.553 92.456) (end 106.553 101.854) (width 0.25) (layer F.Cu) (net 38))
 (segment (start 106.553 101.854) (end 106.807 102.108) (width 0.25) (layer F.Cu) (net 38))
 (segment (start 124.6124 113.4491) (end 126.3142 113.4491) (width 0.25) (layer F.Cu) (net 38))
 (segment (start 115.12 108.372) (end 115.12 112.464) (width 0.25) (layer F.Cu) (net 38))
 (segment (start 116.1051 113.4491) (end 124.6124 113.4491) (width 0.25) (layer F.Cu) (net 38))
 (segment (start 115.12 112.464) (end 116.1051 113.4491) (width 0.25) (layer F.Cu) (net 38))
 (segment (start 113.4 108.372) (end 115.12 108.372) (width 0.25) (layer F.Cu) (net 38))
 (segment (start 113.4 108.372) (end 113.4 117.083) (width 0.25) (layer F.Cu) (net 38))
 (segment (start 113.4 117.083) (end 113.792 117.475) (width 0.25) (layer F.Cu) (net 38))
 (segment (start 106.807 102.108) (end 106.807 102.287) (width 0.25) (layer F.Cu) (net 38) (status 30))
 (segment (start 106.807 102.287) (end 113.4 108.372) (width 0.25) (layer F.Cu) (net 38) (status 10))
 (segment (start 161.29 113.3856) (end 161.29 111.252) (width 0.25) (layer F.Cu) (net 39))
 (segment (start 161.608 110.934) (end 163.576 110.934) (width 0.25) (layer F.Cu) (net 39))
 (segment (start 161.29 111.252) (end 161.608 110.934) (width 0.25) (layer F.Cu) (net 39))
 (segment (start 135.128 118.11) (end 134.366 118.872) (width 0.25) (layer F.Cu) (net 42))
 (segment (start 135.128 112.776) (end 135.128 118.11) (width 0.25) (layer F.Cu) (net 42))
 (segment (start 140.716 107.188) (end 135.128 112.776) (width 0.25) (layer F.Cu) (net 42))
 (via (at 140.716 107.188) (size 0.6) (drill 0.4) (layers F.Cu B.Cu) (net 42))
 (segment (start 145.288 107.188) (end 140.716 107.188) (width 0.25) (layer B.Cu) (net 42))
 (segment (start 145.542 106.934) (end 145.288 107.188) (width 0.25) (layer B.Cu) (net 42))
 (via (at 145.542 106.934) (size 0.6) (drill 0.4) (layers F.Cu B.Cu) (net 42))
 (segment (start 129.7178 113.4491) (end 129.7178 118.7958) (width 0.25) (layer F.Cu) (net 42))
 (segment (start 129.7178 118.7958) (end 130.81 119.888) (width 0.25) (layer F.Cu) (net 42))
 (segment (start 163.576 106.934) (end 145.542 106.934) (width 0.25) (layer F.Cu) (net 42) (status 10))
 (segment (start 134.366 118.872) (end 132.81 119.888) (width 0.25) (layer F.Cu) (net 42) (status 20))
 (segment (start 130.9878 119.7102) (end 130.81 119.888) (width 0.25) (layer F.Cu) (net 42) (status 30))
 (segment (start 130.81 119.888) (end 132.81 119.888) (width 0.25) (layer F.Cu) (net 42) (status 30))
 (segment (start 161.29 114.4016) (end 162.1084 114.4016) (width 0.25) (layer F.Cu) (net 40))
 (segment (start 162.1084 114.4016) (end 163.576 112.934) (width 0.25) (layer F.Cu) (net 40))
 (segment (start 161.29 115.4176) (end 163.0924 115.4176) (width 0.25) (layer F.Cu) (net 41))
 (segment (start 163.0924 115.4176) (end 163.576 114.934) (width 0.25) (layer F.Cu) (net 41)))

